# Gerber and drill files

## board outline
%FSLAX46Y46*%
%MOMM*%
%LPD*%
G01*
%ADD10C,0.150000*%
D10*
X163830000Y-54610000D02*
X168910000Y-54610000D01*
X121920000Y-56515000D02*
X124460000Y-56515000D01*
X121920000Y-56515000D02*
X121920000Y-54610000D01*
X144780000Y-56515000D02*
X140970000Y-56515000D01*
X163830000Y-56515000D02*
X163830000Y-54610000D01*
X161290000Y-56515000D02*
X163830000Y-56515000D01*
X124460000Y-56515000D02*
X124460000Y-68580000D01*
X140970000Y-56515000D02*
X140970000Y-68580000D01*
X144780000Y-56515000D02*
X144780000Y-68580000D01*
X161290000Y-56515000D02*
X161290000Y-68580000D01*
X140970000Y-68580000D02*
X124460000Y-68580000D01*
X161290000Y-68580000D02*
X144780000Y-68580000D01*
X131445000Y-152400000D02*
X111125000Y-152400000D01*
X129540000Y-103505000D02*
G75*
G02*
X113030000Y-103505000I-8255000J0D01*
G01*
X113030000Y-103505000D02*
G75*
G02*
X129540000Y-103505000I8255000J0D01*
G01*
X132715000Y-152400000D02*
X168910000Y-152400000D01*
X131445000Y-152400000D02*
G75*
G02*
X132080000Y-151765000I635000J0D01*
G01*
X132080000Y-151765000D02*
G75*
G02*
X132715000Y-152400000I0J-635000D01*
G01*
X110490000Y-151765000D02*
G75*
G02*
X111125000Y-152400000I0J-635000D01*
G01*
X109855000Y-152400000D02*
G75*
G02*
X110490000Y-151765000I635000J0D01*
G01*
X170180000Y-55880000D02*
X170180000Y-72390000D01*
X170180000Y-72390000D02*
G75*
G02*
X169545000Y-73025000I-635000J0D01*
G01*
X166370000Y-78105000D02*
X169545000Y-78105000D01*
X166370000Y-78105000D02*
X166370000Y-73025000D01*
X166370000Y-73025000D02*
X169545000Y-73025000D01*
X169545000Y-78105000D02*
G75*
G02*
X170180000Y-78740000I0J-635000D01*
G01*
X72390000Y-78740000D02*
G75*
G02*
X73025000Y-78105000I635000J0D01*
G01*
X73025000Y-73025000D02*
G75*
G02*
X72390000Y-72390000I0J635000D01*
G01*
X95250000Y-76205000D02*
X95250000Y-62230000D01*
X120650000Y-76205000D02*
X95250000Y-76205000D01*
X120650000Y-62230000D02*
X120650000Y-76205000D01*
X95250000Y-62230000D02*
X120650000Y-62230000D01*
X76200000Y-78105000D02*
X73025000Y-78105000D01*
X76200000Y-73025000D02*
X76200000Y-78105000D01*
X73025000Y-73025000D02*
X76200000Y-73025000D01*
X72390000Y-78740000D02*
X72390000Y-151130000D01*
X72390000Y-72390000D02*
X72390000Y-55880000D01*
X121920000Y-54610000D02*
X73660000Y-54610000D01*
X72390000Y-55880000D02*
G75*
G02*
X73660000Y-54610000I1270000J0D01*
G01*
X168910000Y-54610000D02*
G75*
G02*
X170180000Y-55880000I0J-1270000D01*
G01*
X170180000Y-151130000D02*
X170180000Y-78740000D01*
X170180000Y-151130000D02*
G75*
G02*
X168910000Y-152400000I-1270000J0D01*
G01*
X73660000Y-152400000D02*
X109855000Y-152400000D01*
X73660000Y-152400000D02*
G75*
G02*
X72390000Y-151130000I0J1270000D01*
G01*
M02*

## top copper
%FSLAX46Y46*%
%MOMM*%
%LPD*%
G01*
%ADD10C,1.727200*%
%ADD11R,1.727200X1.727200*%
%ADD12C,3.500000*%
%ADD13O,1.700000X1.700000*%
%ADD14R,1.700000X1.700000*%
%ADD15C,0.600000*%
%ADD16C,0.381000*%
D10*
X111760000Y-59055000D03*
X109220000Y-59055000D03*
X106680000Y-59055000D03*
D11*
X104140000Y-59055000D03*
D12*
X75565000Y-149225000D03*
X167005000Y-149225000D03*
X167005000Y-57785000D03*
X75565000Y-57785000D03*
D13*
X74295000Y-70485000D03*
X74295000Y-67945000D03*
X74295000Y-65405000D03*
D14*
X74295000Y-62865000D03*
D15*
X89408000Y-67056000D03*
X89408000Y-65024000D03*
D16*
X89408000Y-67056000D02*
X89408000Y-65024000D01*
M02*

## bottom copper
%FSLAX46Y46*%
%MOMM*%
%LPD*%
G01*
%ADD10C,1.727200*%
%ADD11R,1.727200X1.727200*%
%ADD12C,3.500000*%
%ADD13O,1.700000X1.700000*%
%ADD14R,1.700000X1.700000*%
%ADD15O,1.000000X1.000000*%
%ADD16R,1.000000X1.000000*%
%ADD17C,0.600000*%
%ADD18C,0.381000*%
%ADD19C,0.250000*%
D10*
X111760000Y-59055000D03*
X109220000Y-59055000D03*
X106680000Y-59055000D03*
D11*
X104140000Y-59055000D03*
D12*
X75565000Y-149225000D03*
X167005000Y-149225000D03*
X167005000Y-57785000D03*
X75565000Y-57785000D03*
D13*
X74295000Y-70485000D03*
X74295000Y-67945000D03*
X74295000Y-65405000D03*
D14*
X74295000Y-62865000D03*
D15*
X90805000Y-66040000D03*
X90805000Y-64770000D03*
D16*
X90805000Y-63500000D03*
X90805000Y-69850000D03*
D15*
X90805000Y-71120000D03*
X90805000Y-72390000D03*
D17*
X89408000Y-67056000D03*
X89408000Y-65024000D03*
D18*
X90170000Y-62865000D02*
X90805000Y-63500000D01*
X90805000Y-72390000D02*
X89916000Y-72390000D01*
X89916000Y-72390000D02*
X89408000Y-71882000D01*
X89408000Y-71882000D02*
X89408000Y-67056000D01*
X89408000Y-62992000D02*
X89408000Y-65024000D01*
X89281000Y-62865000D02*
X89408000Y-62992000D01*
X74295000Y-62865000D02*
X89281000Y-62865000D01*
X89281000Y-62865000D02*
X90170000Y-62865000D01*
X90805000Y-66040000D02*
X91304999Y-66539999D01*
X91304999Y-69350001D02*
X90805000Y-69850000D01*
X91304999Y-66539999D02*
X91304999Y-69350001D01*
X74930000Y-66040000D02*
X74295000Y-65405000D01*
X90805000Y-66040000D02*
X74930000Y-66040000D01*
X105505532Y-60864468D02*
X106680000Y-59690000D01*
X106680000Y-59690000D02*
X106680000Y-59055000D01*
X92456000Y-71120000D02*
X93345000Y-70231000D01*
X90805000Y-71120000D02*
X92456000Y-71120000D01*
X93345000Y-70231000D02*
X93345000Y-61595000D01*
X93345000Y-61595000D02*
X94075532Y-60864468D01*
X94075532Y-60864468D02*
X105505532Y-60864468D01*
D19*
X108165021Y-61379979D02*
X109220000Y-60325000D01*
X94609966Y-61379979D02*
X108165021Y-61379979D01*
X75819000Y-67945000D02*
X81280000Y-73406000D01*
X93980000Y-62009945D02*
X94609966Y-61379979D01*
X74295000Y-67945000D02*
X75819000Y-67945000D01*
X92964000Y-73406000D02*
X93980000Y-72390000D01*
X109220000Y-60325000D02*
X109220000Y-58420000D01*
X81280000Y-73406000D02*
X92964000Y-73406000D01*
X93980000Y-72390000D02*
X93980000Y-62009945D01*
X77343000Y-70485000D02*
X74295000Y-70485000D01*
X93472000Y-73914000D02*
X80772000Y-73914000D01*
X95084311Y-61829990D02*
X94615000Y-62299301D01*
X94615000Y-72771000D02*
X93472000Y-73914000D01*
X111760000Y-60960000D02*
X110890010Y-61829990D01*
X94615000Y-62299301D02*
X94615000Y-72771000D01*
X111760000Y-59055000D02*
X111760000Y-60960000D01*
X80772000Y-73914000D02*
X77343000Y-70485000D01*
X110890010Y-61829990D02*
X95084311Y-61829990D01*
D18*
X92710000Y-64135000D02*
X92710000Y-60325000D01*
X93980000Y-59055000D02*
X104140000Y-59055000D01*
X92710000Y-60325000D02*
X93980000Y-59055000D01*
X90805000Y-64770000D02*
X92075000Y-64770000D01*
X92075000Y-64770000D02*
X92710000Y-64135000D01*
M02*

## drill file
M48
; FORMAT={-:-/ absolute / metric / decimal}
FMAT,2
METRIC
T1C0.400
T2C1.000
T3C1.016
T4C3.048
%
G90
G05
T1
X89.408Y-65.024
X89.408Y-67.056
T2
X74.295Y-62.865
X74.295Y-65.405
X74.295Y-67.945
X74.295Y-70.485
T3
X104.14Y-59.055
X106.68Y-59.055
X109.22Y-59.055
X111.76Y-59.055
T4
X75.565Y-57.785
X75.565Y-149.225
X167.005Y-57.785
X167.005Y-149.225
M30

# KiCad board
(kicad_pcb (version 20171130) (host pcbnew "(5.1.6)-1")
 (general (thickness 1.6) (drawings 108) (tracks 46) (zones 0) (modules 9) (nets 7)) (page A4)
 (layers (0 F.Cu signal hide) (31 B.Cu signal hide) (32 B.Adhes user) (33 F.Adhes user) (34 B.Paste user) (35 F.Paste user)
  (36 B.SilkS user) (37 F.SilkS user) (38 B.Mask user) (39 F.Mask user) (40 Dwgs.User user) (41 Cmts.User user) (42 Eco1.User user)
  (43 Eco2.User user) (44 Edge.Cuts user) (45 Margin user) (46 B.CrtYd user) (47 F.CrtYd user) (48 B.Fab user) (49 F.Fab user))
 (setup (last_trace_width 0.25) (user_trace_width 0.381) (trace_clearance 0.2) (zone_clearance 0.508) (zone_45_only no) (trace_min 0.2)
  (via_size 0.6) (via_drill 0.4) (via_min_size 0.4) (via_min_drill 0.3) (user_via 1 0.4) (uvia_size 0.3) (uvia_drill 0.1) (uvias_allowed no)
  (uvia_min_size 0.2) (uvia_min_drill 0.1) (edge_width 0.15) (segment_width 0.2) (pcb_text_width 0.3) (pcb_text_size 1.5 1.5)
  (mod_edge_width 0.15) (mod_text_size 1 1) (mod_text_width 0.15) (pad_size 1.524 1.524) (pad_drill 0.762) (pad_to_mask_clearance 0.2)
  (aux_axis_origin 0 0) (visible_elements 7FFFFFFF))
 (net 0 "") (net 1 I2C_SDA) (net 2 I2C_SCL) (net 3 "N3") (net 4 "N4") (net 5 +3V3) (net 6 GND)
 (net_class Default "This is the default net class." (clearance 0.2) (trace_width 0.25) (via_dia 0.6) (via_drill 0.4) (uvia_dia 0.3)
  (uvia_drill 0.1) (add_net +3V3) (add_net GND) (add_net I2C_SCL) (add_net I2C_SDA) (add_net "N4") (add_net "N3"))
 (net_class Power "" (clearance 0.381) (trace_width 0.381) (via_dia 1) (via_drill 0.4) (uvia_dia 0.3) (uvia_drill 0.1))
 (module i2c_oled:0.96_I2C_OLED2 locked (layer F.Cu) (at 107.95 59.055)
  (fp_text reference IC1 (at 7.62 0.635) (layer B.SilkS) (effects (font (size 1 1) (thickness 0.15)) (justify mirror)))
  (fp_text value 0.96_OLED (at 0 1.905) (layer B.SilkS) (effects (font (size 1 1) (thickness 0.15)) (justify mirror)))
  (pad 4 thru_hole circle (at 3.81 0) (size 1.7272 1.7272) (drill 1.016) (layers *.Cu *.Mask) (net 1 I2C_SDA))
  (pad 3 thru_hole circle (at 1.27 0) (size 1.7272 1.7272) (drill 1.016) (layers *.Cu *.Mask) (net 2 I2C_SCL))
  (pad 2 thru_hole circle (at -1.27 0) (size 1.7272 1.7272) (drill 1.016) (layers *.Cu *.Mask) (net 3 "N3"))
  (pad 1 thru_hole rect (at -3.81 0) (size 1.7272 1.7272) (drill 1.016) (layers *.Cu *.Mask) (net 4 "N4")))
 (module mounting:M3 (layer F.Cu) (at 75.565 149.225)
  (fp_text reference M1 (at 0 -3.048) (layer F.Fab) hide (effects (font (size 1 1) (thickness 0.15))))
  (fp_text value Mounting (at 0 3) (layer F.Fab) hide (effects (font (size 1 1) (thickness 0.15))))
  (pad "" np_thru_hole circle (at 0 0) (size 3.5 3.5) (drill 3.048) (layers *.Cu *.Mask) (solder_mask_margin 0.8)))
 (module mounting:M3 (layer F.Cu) (at 167.005 149.225)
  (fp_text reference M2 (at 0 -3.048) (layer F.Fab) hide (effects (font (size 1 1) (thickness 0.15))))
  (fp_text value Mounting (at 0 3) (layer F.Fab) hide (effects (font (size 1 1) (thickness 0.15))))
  (pad "" np_thru_hole circle (at 0 0) (size 3.5 3.5) (drill 3.048) (layers *.Cu *.Mask) (solder_mask_margin 0.8)))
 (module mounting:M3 (layer F.Cu) (at 167.005 57.785)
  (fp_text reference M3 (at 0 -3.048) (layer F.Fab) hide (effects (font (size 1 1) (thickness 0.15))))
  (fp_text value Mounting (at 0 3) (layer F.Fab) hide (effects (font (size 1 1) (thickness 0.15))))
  (pad "" np_thru_hole circle (at 0 0) (size 3.5 3.5) (drill 3.048) (layers *.Cu *.Mask) (solder_mask_margin 0.8)))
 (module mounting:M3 (layer F.Cu) (at 75.565 57.785)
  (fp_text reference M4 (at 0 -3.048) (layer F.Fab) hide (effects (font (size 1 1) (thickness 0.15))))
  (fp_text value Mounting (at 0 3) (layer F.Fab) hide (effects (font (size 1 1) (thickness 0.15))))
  (pad "" np_thru_hole circle (at 0 0) (size 3.5 3.5) (drill 3.048) (layers *.Cu *.Mask) (solder_mask_margin 0.8)))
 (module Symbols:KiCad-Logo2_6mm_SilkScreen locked (layer B.Cu) (at 151.875 91.55 180)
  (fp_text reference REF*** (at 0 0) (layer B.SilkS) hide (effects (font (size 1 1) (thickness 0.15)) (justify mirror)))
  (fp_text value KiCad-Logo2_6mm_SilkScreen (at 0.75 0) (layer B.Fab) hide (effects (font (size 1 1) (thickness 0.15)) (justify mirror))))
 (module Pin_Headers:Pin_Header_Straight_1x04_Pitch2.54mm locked (layer B.Cu) (at 74.295 62.865 180)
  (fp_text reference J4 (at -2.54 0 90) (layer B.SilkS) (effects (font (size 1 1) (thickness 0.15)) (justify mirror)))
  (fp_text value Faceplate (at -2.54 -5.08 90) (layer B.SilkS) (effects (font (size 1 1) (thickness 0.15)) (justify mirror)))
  (pad 4 thru_hole oval (at 0 -7.62 180) (size 1.7 1.7) (drill 1) (layers *.Cu *.Mask) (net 1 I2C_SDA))
  (pad 3 thru_hole oval (at 0 -5.08 180) (size 1.7 1.7) (drill 1) (layers *.Cu *.Mask) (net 2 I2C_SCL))
  (pad 2 thru_hole oval (at 0 -2.54 180) (size 1.7 1.7) (drill 1) (layers *.Cu *.Mask) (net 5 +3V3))
  (pad 1 thru_hole rect (at 0 0 180) (size 1.7 1.7) (drill 1) (layers *.Cu *.Mask) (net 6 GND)))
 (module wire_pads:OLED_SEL (layer B.Cu) (at 90.805 63.5 180)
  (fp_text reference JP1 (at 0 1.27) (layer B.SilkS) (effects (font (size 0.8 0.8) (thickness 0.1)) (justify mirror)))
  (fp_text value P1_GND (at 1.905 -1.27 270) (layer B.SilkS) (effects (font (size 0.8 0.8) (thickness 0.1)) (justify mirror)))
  (pad 3 smd oval (at 0 -2.54 180) (size 1 1) (layers B.Cu B.Paste B.Mask) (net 5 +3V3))
  (pad 2 smd oval (at 0 -1.27 180) (size 1 1) (layers B.Cu B.Paste B.Mask) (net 4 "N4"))
  (pad 1 smd rect (at 0 0 180) (size 1 1) (layers B.Cu B.Paste B.Mask) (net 6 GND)))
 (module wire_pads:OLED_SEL (layer B.Cu) (at 90.805 69.85 180)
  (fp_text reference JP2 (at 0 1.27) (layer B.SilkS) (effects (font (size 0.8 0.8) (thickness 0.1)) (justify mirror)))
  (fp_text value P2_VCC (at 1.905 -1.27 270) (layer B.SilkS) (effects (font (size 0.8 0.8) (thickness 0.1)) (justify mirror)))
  (pad 1 smd rect (at 0 0 180) (size 1 1) (layers B.Cu B.Paste B.Mask) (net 5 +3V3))
  (pad 2 smd oval (at 0 -1.27 180) (size 1 1) (layers B.Cu B.Paste B.Mask) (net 3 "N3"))
  (pad 3 smd oval (at 0 -2.54 180) (size 1 1) (layers B.Cu B.Paste B.Mask) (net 6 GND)))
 (gr_line (start 163.83 54.61) (end 168.91 54.61) (layer Edge.Cuts) (width 0.15))
 (gr_line (start 121.92 56.515) (end 124.46 56.515) (layer Edge.Cuts) (width 0.15))
 (gr_line (start 121.92 56.515) (end 121.92 54.61) (layer Edge.Cuts) (width 0.15))
 (gr_line (start 144.78 56.515) (end 140.97 56.515) (layer Edge.Cuts) (width 0.15))
 (gr_line (start 163.83 56.515) (end 163.83 54.61) (layer Edge.Cuts) (width 0.15))
 (gr_line (start 161.29 56.515) (end 163.83 56.515) (layer Edge.Cuts) (width 0.15))
 (gr_line (start 124.46 56.515) (end 124.46 68.58) (layer Edge.Cuts) (width 0.15))
 (gr_line (start 140.97 56.515) (end 140.97 68.58) (layer Edge.Cuts) (width 0.15))
 (gr_line (start 144.78 56.515) (end 144.78 68.58) (layer Edge.Cuts) (width 0.15))
 (gr_line (start 161.29 56.515) (end 161.29 68.58) (layer Edge.Cuts) (width 0.15))
 (gr_line (start 140.97 68.58) (end 124.46 68.58) (layer Edge.Cuts) (width 0.15))
 (gr_line (start 161.29 68.58) (end 144.78 68.58) (layer Edge.Cuts) (width 0.15))
 (gr_line (start 131.445 152.4) (end 111.125 152.4) (layer Edge.Cuts) (width 0.15))
 (gr_circle (center 121.285 103.505) (end 129.54 103.505) (layer Edge.Cuts) (width 0.15))
 (gr_line (start 132.715 152.4) (end 168.91 152.4) (layer Edge.Cuts) (width 0.15))
 (gr_arc (start 132.08 152.4) (end 132.08 151.765) (angle -90) (layer Edge.Cuts) (width 0.15))
 (gr_arc (start 132.08 152.4) (end 132.715 152.4) (angle -90) (layer Edge.Cuts) (width 0.15))
 (gr_arc (start 110.49 152.4) (end 111.125 152.4) (angle -90) (layer Edge.Cuts) (width 0.15))
 (gr_arc (start 110.49 152.4) (end 110.49 151.765) (angle -90) (layer Edge.Cuts) (width 0.15))
 (gr_line (start 170.18 55.88) (end 170.18 72.39) (layer Edge.Cuts) (width 0.15))
 (gr_arc (start 169.545 72.39) (end 169.545 73.025) (angle -90) (layer Edge.Cuts) (width 0.15))
 (gr_line (start 166.37 78.105) (end 169.545 78.105) (layer Edge.Cuts) (width 0.15))
 (gr_line (start 166.37 78.105) (end 166.37 73.025) (layer Edge.Cuts) (width 0.15))
 (gr_line (start 166.37 73.025) (end 169.545 73.025) (layer Edge.Cuts) (width 0.15))
 (gr_arc (start 169.545 78.74) (end 170.18 78.74) (angle -90) (layer Edge.Cuts) (width 0.15))
 (gr_arc (start 73.025 78.74) (end 73.025 78.105) (angle -90) (layer Edge.Cuts) (width 0.15))
 (gr_arc (start 73.025 72.39) (end 72.39 72.39) (angle -90) (layer Edge.Cuts) (width 0.15))
 (gr_line (start 95.25 76.205) (end 95.25 62.23) (layer Edge.Cuts) (width 0.15))
 (gr_line (start 120.65 76.205) (end 95.25 76.205) (layer Edge.Cuts) (width 0.15))
 (gr_line (start 120.65 62.23) (end 120.65 76.205) (layer Edge.Cuts) (width 0.15))
 (gr_line (start 95.25 62.23) (end 120.65 62.23) (layer Edge.Cuts) (width 0.15))
 (gr_line (start 76.2 78.105) (end 73.025 78.105) (layer Edge.Cuts) (width 0.15))
 (gr_line (start 76.2 73.025) (end 76.2 78.105) (layer Edge.Cuts) (width 0.15))
 (gr_line (start 73.025 73.025) (end 76.2 73.025) (layer Edge.Cuts) (width 0.15))
 (gr_line (start 72.39 78.74) (end 72.39 151.13) (layer Edge.Cuts) (width 0.15))
 (gr_line (start 72.39 72.39) (end 72.39 55.88) (layer Edge.Cuts) (width 0.15))
 (gr_line (start 121.92 54.61) (end 73.66 54.61) (angle 90) (layer Edge.Cuts) (width 0.15))
 (gr_arc (start 73.66 55.88) (end 72.39 55.88) (angle 90) (layer Edge.Cuts) (width 0.15))
 (gr_arc (start 168.91 55.88) (end 168.91 54.61) (angle 90) (layer Edge.Cuts) (width 0.15))
 (gr_line (start 170.18 151.13) (end 170.18 78.74) (angle 90) (layer Edge.Cuts) (width 0.15))
 (gr_arc (start 168.91 151.13) (end 170.18 151.13) (angle 90) (layer Edge.Cuts) (width 0.15))
 (gr_line (start 73.66 152.4) (end 109.855 152.4) (angle 90) (layer Edge.Cuts) (width 0.15))
 (gr_arc (start 73.66 151.13) (end 73.66 152.4) (angle 90) (layer Edge.Cuts) (width 0.15))
 (segment (start 90.17 62.865) (end 90.805 63.5) (width 0.381) (layer B.Cu) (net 6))
 (segment (start 90.805 72.39) (end 89.916 72.39) (width 0.381) (layer B.Cu) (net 6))
 (via (at 89.408 67.056) (size 0.6) (drill 0.4) (layers F.Cu B.Cu) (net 6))
 (segment (start 89.916 72.39) (end 89.408 71.882) (width 0.381) (layer B.Cu) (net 6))
 (segment (start 89.408 71.882) (end 89.408 67.056) (width 0.381) (layer B.Cu) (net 6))
 (via (at 89.408 65.024) (size 0.6) (drill 0.4) (layers F.Cu B.Cu) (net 6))
 (segment (start 89.408 67.056) (end 89.408 65.024) (width 0.381) (layer F.Cu) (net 6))
 (segment (start 89.408 62.992) (end 89.408 65.024) (width 0.381) (layer B.Cu) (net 6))
 (segment (start 89.281 62.865) (end 89.408 62.992) (width 0.381) (layer B.Cu) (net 6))
 (segment (start 74.295 62.865) (end 89.281 62.865) (width 0.381) (layer B.Cu) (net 6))
 (segment (start 89.281 62.865) (end 90.17 62.865) (width 0.381) (layer B.Cu) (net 6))
 (segment (start 90.805 66.04) (end 91.304999 66.539999) (width 0.381) (layer B.Cu) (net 5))
 (segment (start 91.304999 69.350001) (end 90.805 69.85) (width 0.381) (layer B.Cu) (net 5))
 (segment (start 91.304999 66.539999) (end 91.304999 69.350001) (width 0.381) (layer B.Cu) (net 5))
 (segment (start 74.93 66.04) (end 74.295 65.405) (width 0.381) (layer B.Cu) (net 5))
 (segment (start 90.805 66.04) (end 74.93 66.04) (width 0.381) (layer B.Cu) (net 5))
 (segment (start 105.505532 60.864468) (end 106.68 59.69) (width 0.381) (layer B.Cu) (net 3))
 (segment (start 106.68 59.69) (end 106.68 59.055) (width 0.381) (layer B.Cu) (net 3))
 (segment (start 92.456 71.12) (end 93.345 70.231) (width 0.381) (layer B.Cu) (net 3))
 (segment (start 90.805 71.12) (end 92.456 71.12) (width 0.381) (layer B.Cu) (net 3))
 (segment (start 93.345 70.231) (end 93.345 61.595) (width 0.381) (layer B.Cu) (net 3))
 (segment (start 93.345 61.595) (end 94.075532 60.864468) (width 0.381) (layer B.Cu) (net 3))
 (segment (start 94.075532 60.864468) (end 105.505532 60.864468) (width 0.381) (layer B.Cu) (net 3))
 (segment (start 108.165021 61.379979) (end 109.22 60.325) (width 0.25) (layer B.Cu) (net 2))
 (segment (start 94.609966 61.379979) (end 108.165021 61.379979) (width 0.25) (layer B.Cu) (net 2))
 (segment (start 75.819 67.945) (end 81.28 73.406) (width 0.25) (layer B.Cu) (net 2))
 (segment (start 93.98 62.009945) (end 94.609966 61.379979) (width 0.25) (layer B.Cu) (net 2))
 (segment (start 74.295 67.945) (end 75.819 67.945) (width 0.25) (layer B.Cu) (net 2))
 (segment (start 92.964 73.406) (end 93.98 72.39) (width 0.25) (layer B.Cu) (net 2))
 (segment (start 109.22 60.325) (end 109.22 58.42) (width 0.25) (layer B.Cu) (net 2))
 (segment (start 81.28 73.406) (end 92.964 73.406) (width 0.25) (layer B.Cu) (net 2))
 (segment (start 93.98 72.39) (end 93.98 62.009945) (width 0.25) (layer B.Cu) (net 2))
 (segment (start 77.343 70.485) (end 74.295 70.485) (width 0.25) (layer B.Cu) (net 1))
 (segment (start 93.472 73.914) (end 80.772 73.914) (width 0.25) (layer B.Cu) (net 1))
 (segment (start 95.084311 61.82999) (end 94.615 62.299301) (width 0.25) (layer B.Cu) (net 1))
 (segment (start 94.615 72.771) (end 93.472 73.914) (width 0.25) (layer B.Cu) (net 1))
 (segment (start 111.76 60.96) (end 110.89001 61.82999) (width 0.25) (layer B.Cu) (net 1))
 (segment (start 94.615 62.299301) (end 94.615 72.771) (width 0.25) (layer B.Cu) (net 1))
 (segment (start 111.76 59.055) (end 111.76 60.96) (width 0.25) (layer B.Cu) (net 1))
 (segment (start 80.772 73.914) (end 77.343 70.485) (width 0.25) (layer B.Cu) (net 1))
 (segment (start 110.89001 61.82999) (end 95.084311 61.82999) (width 0.25) (layer B.Cu) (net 1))
 (segment (start 92.71 64.135) (end 92.71 60.325) (width 0.381) (layer B.Cu) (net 4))
 (segment (start 93.98 59.055) (end 104.14 59.055) (width 0.381) (layer B.Cu) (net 4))
 (segment (start 92.71 60.325) (end 93.98 59.055) (width 0.381) (layer B.Cu) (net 4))
 (segment (start 90.805 64.77) (end 92.075 64.77) (width 0.381) (layer B.Cu) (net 4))
 (segment (start 92.075 64.77) (end 92.71 64.135) (width 0.381) (layer B.Cu) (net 4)))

